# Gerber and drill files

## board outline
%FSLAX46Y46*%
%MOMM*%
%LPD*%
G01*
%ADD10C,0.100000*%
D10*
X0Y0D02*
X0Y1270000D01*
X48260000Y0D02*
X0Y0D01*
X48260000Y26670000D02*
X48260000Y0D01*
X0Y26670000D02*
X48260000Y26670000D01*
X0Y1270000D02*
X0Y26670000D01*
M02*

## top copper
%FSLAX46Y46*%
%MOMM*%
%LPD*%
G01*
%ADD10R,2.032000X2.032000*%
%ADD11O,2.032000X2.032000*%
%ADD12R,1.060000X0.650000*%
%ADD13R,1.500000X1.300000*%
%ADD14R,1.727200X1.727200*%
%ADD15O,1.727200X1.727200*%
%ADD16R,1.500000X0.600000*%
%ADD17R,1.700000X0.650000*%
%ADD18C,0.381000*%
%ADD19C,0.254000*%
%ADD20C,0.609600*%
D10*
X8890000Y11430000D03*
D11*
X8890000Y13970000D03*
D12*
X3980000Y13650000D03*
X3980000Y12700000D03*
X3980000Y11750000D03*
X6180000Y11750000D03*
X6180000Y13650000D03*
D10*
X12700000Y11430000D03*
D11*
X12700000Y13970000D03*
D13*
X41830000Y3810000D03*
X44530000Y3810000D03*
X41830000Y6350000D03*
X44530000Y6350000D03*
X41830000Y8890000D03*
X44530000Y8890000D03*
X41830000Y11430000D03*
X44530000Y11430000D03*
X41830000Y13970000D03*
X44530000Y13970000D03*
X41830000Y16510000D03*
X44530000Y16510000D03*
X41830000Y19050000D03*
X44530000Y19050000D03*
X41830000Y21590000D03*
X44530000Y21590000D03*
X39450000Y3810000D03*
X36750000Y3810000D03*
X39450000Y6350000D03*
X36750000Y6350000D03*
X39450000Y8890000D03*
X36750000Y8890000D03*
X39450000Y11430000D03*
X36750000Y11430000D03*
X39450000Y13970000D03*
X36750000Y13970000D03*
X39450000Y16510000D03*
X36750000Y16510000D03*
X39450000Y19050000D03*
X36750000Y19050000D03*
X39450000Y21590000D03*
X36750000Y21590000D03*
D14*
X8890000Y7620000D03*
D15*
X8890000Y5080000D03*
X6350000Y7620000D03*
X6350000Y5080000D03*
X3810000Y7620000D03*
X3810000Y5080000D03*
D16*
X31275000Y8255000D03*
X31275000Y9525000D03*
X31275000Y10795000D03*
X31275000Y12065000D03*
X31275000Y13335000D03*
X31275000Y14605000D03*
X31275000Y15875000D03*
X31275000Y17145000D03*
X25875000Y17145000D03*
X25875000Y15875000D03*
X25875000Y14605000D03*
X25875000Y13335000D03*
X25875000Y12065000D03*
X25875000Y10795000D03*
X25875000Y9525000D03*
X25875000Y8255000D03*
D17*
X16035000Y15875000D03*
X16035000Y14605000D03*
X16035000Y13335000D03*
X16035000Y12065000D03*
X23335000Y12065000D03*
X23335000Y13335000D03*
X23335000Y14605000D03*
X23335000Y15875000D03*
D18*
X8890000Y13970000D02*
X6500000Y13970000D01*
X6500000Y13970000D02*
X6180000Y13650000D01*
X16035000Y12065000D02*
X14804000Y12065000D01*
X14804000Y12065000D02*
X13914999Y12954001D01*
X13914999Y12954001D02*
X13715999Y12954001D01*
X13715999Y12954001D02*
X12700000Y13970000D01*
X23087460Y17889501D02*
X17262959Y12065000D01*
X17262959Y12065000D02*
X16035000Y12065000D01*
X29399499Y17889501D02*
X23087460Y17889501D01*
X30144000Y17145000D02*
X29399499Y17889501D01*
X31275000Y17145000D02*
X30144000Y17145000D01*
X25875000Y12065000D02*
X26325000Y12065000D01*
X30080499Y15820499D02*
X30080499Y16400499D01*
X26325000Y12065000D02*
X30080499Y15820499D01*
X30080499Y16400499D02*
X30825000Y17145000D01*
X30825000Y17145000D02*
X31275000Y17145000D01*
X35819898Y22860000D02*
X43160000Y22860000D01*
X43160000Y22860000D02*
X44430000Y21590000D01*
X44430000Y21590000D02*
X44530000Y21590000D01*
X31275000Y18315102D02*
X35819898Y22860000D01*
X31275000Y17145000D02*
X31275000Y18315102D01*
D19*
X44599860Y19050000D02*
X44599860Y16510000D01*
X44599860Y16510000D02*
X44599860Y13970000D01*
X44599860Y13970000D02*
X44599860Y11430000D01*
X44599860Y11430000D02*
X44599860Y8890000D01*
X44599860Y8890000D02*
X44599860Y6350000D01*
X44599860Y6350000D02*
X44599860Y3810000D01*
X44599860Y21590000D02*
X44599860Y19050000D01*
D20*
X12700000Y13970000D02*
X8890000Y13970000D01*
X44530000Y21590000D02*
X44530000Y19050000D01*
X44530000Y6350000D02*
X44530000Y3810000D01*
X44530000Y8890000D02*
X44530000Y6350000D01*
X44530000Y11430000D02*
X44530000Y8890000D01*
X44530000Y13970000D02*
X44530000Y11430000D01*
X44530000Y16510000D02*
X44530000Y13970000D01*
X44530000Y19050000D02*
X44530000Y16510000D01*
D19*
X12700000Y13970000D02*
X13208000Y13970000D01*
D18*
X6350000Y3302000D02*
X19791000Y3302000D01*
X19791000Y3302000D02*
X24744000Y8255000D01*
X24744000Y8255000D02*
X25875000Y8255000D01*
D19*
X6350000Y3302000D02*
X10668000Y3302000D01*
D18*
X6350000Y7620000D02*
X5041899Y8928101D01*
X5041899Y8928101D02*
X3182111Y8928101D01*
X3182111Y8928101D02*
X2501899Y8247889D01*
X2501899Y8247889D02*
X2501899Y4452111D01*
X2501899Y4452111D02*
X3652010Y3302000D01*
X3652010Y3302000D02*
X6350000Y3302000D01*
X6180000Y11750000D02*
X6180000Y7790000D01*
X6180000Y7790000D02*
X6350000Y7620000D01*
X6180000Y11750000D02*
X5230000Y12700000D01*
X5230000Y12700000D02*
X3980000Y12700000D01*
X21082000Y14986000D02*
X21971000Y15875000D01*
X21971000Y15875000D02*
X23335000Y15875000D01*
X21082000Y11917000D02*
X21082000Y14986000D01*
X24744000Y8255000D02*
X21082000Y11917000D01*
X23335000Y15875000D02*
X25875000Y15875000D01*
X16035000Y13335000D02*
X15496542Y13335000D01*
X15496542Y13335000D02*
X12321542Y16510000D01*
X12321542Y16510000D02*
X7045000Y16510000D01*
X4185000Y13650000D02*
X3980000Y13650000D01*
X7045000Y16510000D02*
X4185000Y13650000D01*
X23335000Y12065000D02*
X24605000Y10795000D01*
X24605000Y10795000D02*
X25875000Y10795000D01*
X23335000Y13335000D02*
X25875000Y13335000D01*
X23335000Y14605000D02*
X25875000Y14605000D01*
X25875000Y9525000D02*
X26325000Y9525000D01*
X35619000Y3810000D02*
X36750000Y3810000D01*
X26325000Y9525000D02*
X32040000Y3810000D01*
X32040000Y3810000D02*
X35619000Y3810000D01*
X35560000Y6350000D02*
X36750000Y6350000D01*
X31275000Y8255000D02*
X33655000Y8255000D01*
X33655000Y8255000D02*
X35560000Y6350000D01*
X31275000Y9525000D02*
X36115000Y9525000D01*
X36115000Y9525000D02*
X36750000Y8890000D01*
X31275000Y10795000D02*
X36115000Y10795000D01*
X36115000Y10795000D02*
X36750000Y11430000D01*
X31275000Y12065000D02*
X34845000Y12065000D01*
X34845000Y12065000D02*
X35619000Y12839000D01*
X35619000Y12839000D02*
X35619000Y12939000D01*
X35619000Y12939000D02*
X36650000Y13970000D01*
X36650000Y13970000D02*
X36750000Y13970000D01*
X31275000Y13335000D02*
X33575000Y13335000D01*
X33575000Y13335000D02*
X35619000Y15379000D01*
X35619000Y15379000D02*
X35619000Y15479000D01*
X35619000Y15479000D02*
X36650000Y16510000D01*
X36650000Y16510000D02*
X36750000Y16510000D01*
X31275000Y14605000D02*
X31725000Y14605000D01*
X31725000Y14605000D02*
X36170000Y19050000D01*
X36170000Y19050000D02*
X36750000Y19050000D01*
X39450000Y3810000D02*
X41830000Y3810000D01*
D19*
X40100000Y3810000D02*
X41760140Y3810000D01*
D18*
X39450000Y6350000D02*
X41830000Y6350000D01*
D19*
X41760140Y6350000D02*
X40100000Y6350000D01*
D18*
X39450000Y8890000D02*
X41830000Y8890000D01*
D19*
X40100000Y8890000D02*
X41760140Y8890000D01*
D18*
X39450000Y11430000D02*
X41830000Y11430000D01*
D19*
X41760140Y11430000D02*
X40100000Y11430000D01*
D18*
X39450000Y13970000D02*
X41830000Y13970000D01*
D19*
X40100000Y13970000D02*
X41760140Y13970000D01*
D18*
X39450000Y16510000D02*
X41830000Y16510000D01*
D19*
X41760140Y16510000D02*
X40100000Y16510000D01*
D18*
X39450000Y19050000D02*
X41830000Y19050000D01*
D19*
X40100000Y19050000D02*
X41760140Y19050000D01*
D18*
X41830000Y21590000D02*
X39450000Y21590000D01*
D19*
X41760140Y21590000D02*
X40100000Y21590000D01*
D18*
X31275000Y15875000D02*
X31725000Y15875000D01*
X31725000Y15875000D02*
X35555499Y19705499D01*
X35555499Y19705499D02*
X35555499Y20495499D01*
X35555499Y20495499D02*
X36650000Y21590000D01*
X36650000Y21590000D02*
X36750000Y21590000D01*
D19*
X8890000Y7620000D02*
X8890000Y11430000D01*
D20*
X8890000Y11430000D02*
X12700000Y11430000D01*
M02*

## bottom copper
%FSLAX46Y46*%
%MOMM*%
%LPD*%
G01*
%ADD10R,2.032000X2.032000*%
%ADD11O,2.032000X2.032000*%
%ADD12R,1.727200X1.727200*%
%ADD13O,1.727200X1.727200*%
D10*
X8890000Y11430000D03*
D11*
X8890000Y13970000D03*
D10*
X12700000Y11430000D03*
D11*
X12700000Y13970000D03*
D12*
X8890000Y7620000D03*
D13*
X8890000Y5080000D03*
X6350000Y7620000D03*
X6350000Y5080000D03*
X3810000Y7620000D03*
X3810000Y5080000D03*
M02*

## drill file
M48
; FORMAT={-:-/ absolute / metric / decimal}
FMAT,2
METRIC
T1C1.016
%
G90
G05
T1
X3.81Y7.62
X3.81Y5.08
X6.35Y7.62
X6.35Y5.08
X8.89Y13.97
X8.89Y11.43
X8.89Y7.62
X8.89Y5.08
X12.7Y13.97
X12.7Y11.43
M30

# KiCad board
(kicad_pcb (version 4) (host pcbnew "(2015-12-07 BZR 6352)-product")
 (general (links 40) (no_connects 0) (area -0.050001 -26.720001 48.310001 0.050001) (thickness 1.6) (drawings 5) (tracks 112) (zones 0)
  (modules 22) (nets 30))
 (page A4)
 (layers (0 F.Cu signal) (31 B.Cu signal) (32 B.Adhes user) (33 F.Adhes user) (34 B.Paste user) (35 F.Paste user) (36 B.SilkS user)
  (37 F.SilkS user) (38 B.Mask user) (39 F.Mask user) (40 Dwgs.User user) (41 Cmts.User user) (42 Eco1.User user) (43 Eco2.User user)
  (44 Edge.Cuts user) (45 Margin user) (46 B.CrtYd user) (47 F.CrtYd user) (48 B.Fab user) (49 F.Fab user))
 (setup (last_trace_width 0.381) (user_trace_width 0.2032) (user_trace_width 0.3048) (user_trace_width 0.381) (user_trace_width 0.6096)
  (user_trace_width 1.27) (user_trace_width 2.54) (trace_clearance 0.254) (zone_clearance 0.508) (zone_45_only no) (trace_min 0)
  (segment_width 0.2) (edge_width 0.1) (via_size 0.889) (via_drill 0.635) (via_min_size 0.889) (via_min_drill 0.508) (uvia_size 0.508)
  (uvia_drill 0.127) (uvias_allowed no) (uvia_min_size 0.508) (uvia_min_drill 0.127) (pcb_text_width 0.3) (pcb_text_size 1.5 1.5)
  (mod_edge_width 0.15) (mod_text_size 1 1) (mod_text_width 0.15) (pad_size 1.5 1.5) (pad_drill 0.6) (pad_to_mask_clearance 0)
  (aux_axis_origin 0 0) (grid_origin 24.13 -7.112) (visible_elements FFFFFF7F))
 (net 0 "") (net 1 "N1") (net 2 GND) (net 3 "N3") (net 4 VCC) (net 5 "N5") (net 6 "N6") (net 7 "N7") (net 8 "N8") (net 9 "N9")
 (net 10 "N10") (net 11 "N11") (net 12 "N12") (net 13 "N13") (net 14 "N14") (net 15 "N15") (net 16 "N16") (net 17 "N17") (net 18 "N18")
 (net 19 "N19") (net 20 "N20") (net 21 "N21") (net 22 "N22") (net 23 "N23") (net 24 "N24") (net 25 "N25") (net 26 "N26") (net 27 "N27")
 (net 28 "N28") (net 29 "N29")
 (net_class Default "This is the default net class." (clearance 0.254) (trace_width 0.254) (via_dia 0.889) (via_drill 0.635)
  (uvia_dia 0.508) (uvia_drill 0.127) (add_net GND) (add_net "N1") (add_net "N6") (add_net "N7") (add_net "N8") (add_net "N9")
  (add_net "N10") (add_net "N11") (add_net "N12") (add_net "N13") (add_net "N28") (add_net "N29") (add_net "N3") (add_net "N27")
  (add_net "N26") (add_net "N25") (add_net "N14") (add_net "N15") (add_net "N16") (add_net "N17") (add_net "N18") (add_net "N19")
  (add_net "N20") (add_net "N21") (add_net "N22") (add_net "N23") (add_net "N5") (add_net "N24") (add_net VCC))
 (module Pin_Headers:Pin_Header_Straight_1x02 (layer F.Cu) (at 8.89 -11.43 180)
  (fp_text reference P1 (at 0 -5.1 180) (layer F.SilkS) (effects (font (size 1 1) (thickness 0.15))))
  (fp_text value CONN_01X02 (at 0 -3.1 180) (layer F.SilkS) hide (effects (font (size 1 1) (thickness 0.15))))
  (pad 1 thru_hole rect (at 0 0 180) (size 2.032 2.032) (drill 1.016) (layers *.Cu *.Mask F.SilkS) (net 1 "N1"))
  (pad 2 thru_hole oval (at 0 2.54 180) (size 2.032 2.032) (drill 1.016) (layers *.Cu *.Mask F.SilkS) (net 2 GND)))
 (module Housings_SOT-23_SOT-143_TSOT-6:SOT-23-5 (layer F.Cu) (at 5.08 -12.7)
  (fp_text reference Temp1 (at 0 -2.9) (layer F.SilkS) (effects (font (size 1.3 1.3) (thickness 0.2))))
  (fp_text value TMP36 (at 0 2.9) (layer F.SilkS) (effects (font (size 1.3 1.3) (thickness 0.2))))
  (pad 1 smd rect (at -1.1 -0.95) (size 1.06 0.65) (layers F.Cu F.Paste F.Mask) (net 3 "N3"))
  (pad 2 smd rect (at -1.1 0) (size 1.06 0.65) (layers F.Cu F.Paste F.Mask) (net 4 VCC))
  (pad 3 smd rect (at -1.1 0.95) (size 1.06 0.65) (layers F.Cu F.Paste F.Mask) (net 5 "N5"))
  (pad 4 smd rect (at 1.1 0.95) (size 1.06 0.65) (layers F.Cu F.Paste F.Mask) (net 4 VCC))
  (pad 5 smd rect (at 1.1 -0.95) (size 1.06 0.65) (layers F.Cu F.Paste F.Mask) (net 2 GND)))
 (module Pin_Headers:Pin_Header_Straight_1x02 (layer F.Cu) (at 12.7 -11.43 180)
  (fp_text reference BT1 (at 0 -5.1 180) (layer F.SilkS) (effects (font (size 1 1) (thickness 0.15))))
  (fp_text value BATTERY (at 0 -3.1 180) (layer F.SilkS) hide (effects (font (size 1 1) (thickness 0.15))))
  (pad 1 thru_hole rect (at 0 0 180) (size 2.032 2.032) (drill 1.016) (layers *.Cu *.Mask F.SilkS) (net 1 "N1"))
  (pad 2 thru_hole oval (at 0 2.54 180) (size 2.032 2.032) (drill 1.016) (layers *.Cu *.Mask F.SilkS) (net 2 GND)))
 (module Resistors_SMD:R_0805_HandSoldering (layer F.Cu) (at 43.18 -3.81)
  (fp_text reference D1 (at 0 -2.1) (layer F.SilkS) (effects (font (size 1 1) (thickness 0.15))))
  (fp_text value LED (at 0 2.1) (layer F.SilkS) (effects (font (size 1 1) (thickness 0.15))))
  (pad 1 smd rect (at -1.35 0) (size 1.5 1.3) (layers F.Cu F.Paste F.Mask) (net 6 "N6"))
  (pad 2 smd rect (at 1.35 0) (size 1.5 1.3) (layers F.Cu F.Paste F.Mask) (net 2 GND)))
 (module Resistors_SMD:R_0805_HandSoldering (layer F.Cu) (at 43.18 -6.35)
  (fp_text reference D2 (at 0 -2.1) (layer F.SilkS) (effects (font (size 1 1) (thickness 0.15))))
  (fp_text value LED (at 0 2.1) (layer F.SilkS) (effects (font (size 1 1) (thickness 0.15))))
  (pad 1 smd rect (at -1.35 0) (size 1.5 1.3) (layers F.Cu F.Paste F.Mask) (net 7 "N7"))
  (pad 2 smd rect (at 1.35 0) (size 1.5 1.3) (layers F.Cu F.Paste F.Mask) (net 2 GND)))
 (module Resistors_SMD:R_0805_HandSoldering (layer F.Cu) (at 43.18 -8.89)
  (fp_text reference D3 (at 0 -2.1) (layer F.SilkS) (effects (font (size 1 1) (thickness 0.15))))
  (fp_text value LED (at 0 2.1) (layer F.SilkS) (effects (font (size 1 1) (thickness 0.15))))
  (pad 1 smd rect (at -1.35 0) (size 1.5 1.3) (layers F.Cu F.Paste F.Mask) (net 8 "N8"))
  (pad 2 smd rect (at 1.35 0) (size 1.5 1.3) (layers F.Cu F.Paste F.Mask) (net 2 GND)))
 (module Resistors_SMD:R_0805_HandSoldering (layer F.Cu) (at 43.18 -11.43)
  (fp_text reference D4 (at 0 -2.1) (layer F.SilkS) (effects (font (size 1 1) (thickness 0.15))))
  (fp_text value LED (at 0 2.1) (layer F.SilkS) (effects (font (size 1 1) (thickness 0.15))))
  (pad 1 smd rect (at -1.35 0) (size 1.5 1.3) (layers F.Cu F.Paste F.Mask) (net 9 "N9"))
  (pad 2 smd rect (at 1.35 0) (size 1.5 1.3) (layers F.Cu F.Paste F.Mask) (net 2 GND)))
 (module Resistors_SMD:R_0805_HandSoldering (layer F.Cu) (at 43.18 -13.97)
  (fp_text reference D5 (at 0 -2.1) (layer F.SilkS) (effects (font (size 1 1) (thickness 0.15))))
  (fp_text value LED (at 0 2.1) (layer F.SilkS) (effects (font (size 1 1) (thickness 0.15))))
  (pad 1 smd rect (at -1.35 0) (size 1.5 1.3) (layers F.Cu F.Paste F.Mask) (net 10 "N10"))
  (pad 2 smd rect (at 1.35 0) (size 1.5 1.3) (layers F.Cu F.Paste F.Mask) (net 2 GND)))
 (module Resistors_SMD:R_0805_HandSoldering (layer F.Cu) (at 43.18 -16.51)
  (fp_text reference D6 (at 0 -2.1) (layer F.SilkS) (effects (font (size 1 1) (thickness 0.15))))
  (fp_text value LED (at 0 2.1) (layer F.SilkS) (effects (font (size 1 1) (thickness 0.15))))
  (pad 1 smd rect (at -1.35 0) (size 1.5 1.3) (layers F.Cu F.Paste F.Mask) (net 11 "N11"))
  (pad 2 smd rect (at 1.35 0) (size 1.5 1.3) (layers F.Cu F.Paste F.Mask) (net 2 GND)))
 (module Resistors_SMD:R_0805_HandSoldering (layer F.Cu) (at 43.18 -19.05)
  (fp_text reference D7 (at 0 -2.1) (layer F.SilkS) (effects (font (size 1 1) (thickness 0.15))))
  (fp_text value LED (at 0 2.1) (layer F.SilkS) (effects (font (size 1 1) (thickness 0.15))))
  (pad 1 smd rect (at -1.35 0) (size 1.5 1.3) (layers F.Cu F.Paste F.Mask) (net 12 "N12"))
  (pad 2 smd rect (at 1.35 0) (size 1.5 1.3) (layers F.Cu F.Paste F.Mask) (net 2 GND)))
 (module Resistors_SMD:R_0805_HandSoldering (layer F.Cu) (at 43.18 -21.59)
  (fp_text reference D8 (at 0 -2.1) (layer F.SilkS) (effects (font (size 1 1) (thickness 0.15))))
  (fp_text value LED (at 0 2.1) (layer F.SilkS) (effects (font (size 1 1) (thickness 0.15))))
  (pad 1 smd rect (at -1.35 0) (size 1.5 1.3) (layers F.Cu F.Paste F.Mask) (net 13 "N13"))
  (pad 2 smd rect (at 1.35 0) (size 1.5 1.3) (layers F.Cu F.Paste F.Mask) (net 2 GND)))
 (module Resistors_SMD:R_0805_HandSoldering (layer F.Cu) (at 38.1 -3.81 180)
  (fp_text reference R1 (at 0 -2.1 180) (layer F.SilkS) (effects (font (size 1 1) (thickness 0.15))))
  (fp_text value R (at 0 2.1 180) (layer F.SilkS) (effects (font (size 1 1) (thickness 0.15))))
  (pad 1 smd rect (at -1.35 0 180) (size 1.5 1.3) (layers F.Cu F.Paste F.Mask) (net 6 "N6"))
  (pad 2 smd rect (at 1.35 0 180) (size 1.5 1.3) (layers F.Cu F.Paste F.Mask) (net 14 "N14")))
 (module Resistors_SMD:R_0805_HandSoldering (layer F.Cu) (at 38.1 -6.35 180)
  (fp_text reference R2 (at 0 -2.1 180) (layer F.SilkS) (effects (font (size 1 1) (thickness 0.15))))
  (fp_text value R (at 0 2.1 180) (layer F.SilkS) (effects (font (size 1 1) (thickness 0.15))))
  (pad 1 smd rect (at -1.35 0 180) (size 1.5 1.3) (layers F.Cu F.Paste F.Mask) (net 7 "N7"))
  (pad 2 smd rect (at 1.35 0 180) (size 1.5 1.3) (layers F.Cu F.Paste F.Mask) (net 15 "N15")))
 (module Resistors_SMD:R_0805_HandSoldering (layer F.Cu) (at 38.1 -8.89 180)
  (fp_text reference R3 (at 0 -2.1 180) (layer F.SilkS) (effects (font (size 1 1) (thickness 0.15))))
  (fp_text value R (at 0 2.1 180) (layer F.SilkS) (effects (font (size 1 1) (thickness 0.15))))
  (pad 1 smd rect (at -1.35 0 180) (size 1.5 1.3) (layers F.Cu F.Paste F.Mask) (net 8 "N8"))
  (pad 2 smd rect (at 1.35 0 180) (size 1.5 1.3) (layers F.Cu F.Paste F.Mask) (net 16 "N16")))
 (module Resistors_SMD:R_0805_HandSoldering (layer F.Cu) (at 38.1 -11.43 180)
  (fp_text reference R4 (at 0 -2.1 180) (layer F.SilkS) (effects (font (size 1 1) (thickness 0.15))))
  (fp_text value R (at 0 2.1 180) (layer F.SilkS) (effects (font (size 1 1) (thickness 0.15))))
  (pad 1 smd rect (at -1.35 0 180) (size 1.5 1.3) (layers F.Cu F.Paste F.Mask) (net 9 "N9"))
  (pad 2 smd rect (at 1.35 0 180) (size 1.5 1.3) (layers F.Cu F.Paste F.Mask) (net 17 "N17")))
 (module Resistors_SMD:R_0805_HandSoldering (layer F.Cu) (at 38.1 -13.97 180)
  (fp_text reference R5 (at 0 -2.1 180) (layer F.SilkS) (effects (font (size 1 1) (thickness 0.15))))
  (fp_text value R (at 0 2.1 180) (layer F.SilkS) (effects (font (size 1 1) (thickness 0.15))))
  (pad 1 smd rect (at -1.35 0 180) (size 1.5 1.3) (layers F.Cu F.Paste F.Mask) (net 10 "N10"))
  (pad 2 smd rect (at 1.35 0 180) (size 1.5 1.3) (layers F.Cu F.Paste F.Mask) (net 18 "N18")))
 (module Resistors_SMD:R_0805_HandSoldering (layer F.Cu) (at 38.1 -16.51 180)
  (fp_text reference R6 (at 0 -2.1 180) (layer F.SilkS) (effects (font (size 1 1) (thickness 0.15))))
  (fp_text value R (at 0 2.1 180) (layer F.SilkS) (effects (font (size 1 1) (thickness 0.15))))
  (pad 1 smd rect (at -1.35 0 180) (size 1.5 1.3) (layers F.Cu F.Paste F.Mask) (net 11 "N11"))
  (pad 2 smd rect (at 1.35 0 180) (size 1.5 1.3) (layers F.Cu F.Paste F.Mask) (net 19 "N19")))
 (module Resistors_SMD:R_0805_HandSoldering (layer F.Cu) (at 38.1 -19.05 180)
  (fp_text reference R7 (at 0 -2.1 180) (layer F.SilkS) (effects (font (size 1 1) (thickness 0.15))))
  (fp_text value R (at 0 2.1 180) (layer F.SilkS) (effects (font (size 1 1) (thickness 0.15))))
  (pad 1 smd rect (at -1.35 0 180) (size 1.5 1.3) (layers F.Cu F.Paste F.Mask) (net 12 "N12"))
  (pad 2 smd rect (at 1.35 0 180) (size 1.5 1.3) (layers F.Cu F.Paste F.Mask) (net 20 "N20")))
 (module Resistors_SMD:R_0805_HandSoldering (layer F.Cu) (at 38.1 -21.59 180)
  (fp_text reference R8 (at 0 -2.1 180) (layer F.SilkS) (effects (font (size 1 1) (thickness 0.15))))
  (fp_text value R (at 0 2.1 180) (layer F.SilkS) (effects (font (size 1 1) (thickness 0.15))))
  (pad 1 smd rect (at -1.35 0 180) (size 1.5 1.3) (layers F.Cu F.Paste F.Mask) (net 13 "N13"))
  (pad 2 smd rect (at 1.35 0 180) (size 1.5 1.3) (layers F.Cu F.Paste F.Mask) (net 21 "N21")))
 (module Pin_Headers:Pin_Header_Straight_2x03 (layer F.Cu) (at 8.89 -7.62 270)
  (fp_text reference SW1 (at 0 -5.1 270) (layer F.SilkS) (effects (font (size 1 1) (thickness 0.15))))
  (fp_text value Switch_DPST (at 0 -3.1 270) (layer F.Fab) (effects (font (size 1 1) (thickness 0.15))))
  (pad 1 thru_hole rect (at 0 0 270) (size 1.7272 1.7272) (drill 1.016) (layers *.Cu *.Mask F.SilkS) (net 1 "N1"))
  (pad 2 thru_hole oval (at 2.54 0 270) (size 1.7272 1.7272) (drill 1.016) (layers *.Cu *.Mask F.SilkS) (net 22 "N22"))
  (pad 3 thru_hole oval (at 0 2.54 270) (size 1.7272 1.7272) (drill 1.016) (layers *.Cu *.Mask F.SilkS) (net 4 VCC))
  (pad 4 thru_hole oval (at 2.54 2.54 270) (size 1.7272 1.7272) (drill 1.016) (layers *.Cu *.Mask F.SilkS) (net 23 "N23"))
  (pad 5 thru_hole oval (at 0 5.08 270) (size 1.7272 1.7272) (drill 1.016) (layers *.Cu *.Mask F.SilkS))
  (pad 6 thru_hole oval (at 2.54 5.08 270) (size 1.7272 1.7272) (drill 1.016) (layers *.Cu *.Mask F.SilkS)))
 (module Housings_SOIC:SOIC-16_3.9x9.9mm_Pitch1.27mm (layer F.Cu) (at 28.575 -12.7 180)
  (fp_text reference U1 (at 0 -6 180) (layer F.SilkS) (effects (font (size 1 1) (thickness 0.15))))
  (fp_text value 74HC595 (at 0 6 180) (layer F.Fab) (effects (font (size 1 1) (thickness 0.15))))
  (pad 1 smd rect (at -2.7 -4.445 180) (size 1.5 0.6) (layers F.Cu F.Paste F.Mask) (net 15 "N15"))
  (pad 2 smd rect (at -2.7 -3.175 180) (size 1.5 0.6) (layers F.Cu F.Paste F.Mask) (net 16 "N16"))
  (pad 3 smd rect (at -2.7 -1.905 180) (size 1.5 0.6) (layers F.Cu F.Paste F.Mask) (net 17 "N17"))
  (pad 4 smd rect (at -2.7 -0.635 180) (size 1.5 0.6) (layers F.Cu F.Paste F.Mask) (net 18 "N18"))
  (pad 5 smd rect (at -2.7 0.635 180) (size 1.5 0.6) (layers F.Cu F.Paste F.Mask) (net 19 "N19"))
  (pad 6 smd rect (at -2.7 1.905 180) (size 1.5 0.6) (layers F.Cu F.Paste F.Mask) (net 20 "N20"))
  (pad 7 smd rect (at -2.7 3.175 180) (size 1.5 0.6) (layers F.Cu F.Paste F.Mask) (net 21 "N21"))
  (pad 8 smd rect (at -2.7 4.445 180) (size 1.5 0.6) (layers F.Cu F.Paste F.Mask) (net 2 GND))
  (pad 9 smd rect (at 2.7 4.445 180) (size 1.5 0.6) (layers F.Cu F.Paste F.Mask) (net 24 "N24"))
  (pad 10 smd rect (at 2.7 3.175 180) (size 1.5 0.6) (layers F.Cu F.Paste F.Mask) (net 4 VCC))
  (pad 11 smd rect (at 2.7 1.905 180) (size 1.5 0.6) (layers F.Cu F.Paste F.Mask) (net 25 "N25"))
  (pad 12 smd rect (at 2.7 0.635 180) (size 1.5 0.6) (layers F.Cu F.Paste F.Mask) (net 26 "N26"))
  (pad 13 smd rect (at 2.7 -0.635 180) (size 1.5 0.6) (layers F.Cu F.Paste F.Mask) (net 2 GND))
  (pad 14 smd rect (at 2.7 -1.905 180) (size 1.5 0.6) (layers F.Cu F.Paste F.Mask) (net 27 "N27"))
  (pad 15 smd rect (at 2.7 -3.175 180) (size 1.5 0.6) (layers F.Cu F.Paste F.Mask) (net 14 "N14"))
  (pad 16 smd rect (at 2.7 -4.445 180) (size 1.5 0.6) (layers F.Cu F.Paste F.Mask) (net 4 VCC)))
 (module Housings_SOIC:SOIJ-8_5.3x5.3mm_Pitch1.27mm (layer F.Cu) (at 19.685 -13.97)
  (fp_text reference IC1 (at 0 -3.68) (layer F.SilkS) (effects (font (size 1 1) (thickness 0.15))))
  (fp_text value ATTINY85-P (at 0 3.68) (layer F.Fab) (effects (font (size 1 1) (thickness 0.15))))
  (pad 1 smd rect (at -3.65 -1.905) (size 1.7 0.65) (layers F.Cu F.Paste F.Mask) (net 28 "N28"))
  (pad 2 smd rect (at -3.65 -0.635) (size 1.7 0.65) (layers F.Cu F.Paste F.Mask) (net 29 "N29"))
  (pad 3 smd rect (at -3.65 0.635) (size 1.7 0.65) (layers F.Cu F.Paste F.Mask) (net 3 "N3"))
  (pad 4 smd rect (at -3.65 1.905) (size 1.7 0.65) (layers F.Cu F.Paste F.Mask) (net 2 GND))
  (pad 5 smd rect (at 3.65 1.905) (size 1.7 0.65) (layers F.Cu F.Paste F.Mask) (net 27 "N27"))
  (pad 6 smd rect (at 3.65 0.635) (size 1.7 0.65) (layers F.Cu F.Paste F.Mask) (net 26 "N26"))
  (pad 7 smd rect (at 3.65 -0.635) (size 1.7 0.65) (layers F.Cu F.Paste F.Mask) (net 25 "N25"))
  (pad 8 smd rect (at 3.65 -1.905) (size 1.7 0.65) (layers F.Cu F.Paste F.Mask) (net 4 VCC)))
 (gr_line (start 0 0) (end 0 -1.27) (angle 90) (layer Edge.Cuts) (width 0.1))
 (gr_line (start 48.26 0) (end 0 0) (angle 90) (layer Edge.Cuts) (width 0.1))
 (gr_line (start 48.26 -26.67) (end 48.26 0) (angle 90) (layer Edge.Cuts) (width 0.1))
 (gr_line (start 0 -26.67) (end 48.26 -26.67) (angle 90) (layer Edge.Cuts) (width 0.1))
 (gr_line (start 0 -1.27) (end 0 -26.67) (angle 90) (layer Edge.Cuts) (width 0.1))
 (segment (start 8.89 -13.97) (end 6.5 -13.97) (width 0.381) (layer F.Cu) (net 2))
 (segment (start 6.5 -13.97) (end 6.18 -13.65) (width 0.381) (layer F.Cu) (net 2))
 (segment (start 16.035 -12.065) (end 14.804 -12.065) (width 0.381) (layer F.Cu) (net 2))
 (segment (start 14.804 -12.065) (end 13.914999 -12.954001) (width 0.381) (layer F.Cu) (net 2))
 (segment (start 13.914999 -12.954001) (end 13.715999 -12.954001) (width 0.381) (layer F.Cu) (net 2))
 (segment (start 13.715999 -12.954001) (end 12.7 -13.97) (width 0.381) (layer F.Cu) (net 2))
 (segment (start 23.08746 -17.889501) (end 17.262959 -12.065) (width 0.381) (layer F.Cu) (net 2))
 (segment (start 17.262959 -12.065) (end 16.035 -12.065) (width 0.381) (layer F.Cu) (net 2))
 (segment (start 29.399499 -17.889501) (end 23.08746 -17.889501) (width 0.381) (layer F.Cu) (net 2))
 (segment (start 30.144 -17.145) (end 29.399499 -17.889501) (width 0.381) (layer F.Cu) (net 2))
 (segment (start 31.275 -17.145) (end 30.144 -17.145) (width 0.381) (layer F.Cu) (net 2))
 (segment (start 25.875 -12.065) (end 26.325 -12.065) (width 0.381) (layer F.Cu) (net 2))
 (segment (start 30.080499 -15.820499) (end 30.080499 -16.400499) (width 0.381) (layer F.Cu) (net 2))
 (segment (start 26.325 -12.065) (end 30.080499 -15.820499) (width 0.381) (layer F.Cu) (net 2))
 (segment (start 30.080499 -16.400499) (end 30.825 -17.145) (width 0.381) (layer F.Cu) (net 2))
 (segment (start 30.825 -17.145) (end 31.275 -17.145) (width 0.381) (layer F.Cu) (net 2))
 (segment (start 35.819898 -22.86) (end 43.16 -22.86) (width 0.381) (layer F.Cu) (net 2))
 (segment (start 43.16 -22.86) (end 44.43 -21.59) (width 0.381) (layer F.Cu) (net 2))
 (segment (start 44.43 -21.59) (end 44.53 -21.59) (width 0.381) (layer F.Cu) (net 2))
 (segment (start 31.275 -18.315102) (end 35.819898 -22.86) (width 0.381) (layer F.Cu) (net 2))
 (segment (start 31.275 -17.145) (end 31.275 -18.315102) (width 0.381) (layer F.Cu) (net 2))
 (segment (start 44.59986 -19.05) (end 44.59986 -16.51) (width 0.254) (layer F.Cu) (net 2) (status 20))
 (segment (start 44.59986 -16.51) (end 44.59986 -13.97) (width 0.254) (layer F.Cu) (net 2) (status 20))
 (segment (start 44.59986 -13.97) (end 44.59986 -11.43) (width 0.254) (layer F.Cu) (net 2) (status 20))
 (segment (start 44.59986 -11.43) (end 44.59986 -8.89) (width 0.254) (layer F.Cu) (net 2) (status 20))
 (segment (start 44.59986 -8.89) (end 44.59986 -6.35) (width 0.254) (layer F.Cu) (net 2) (status 20))
 (segment (start 44.59986 -6.35) (end 44.59986 -3.81) (width 0.254) (layer F.Cu) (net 2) (status 20))
 (segment (start 44.59986 -21.59) (end 44.59986 -19.05) (width 0.254) (layer F.Cu) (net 2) (status 20))
 (segment (start 12.7 -13.97) (end 8.89 -13.97) (width 0.6096) (layer F.Cu) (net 2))
 (segment (start 44.53 -21.59) (end 44.53 -19.05) (width 0.6096) (layer F.Cu) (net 2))
 (segment (start 44.53 -6.35) (end 44.53 -3.81) (width 0.6096) (layer F.Cu) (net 2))
 (segment (start 44.53 -8.89) (end 44.53 -6.35) (width 0.6096) (layer F.Cu) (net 2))
 (segment (start 44.53 -11.43) (end 44.53 -8.89) (width 0.6096) (layer F.Cu) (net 2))
 (segment (start 44.53 -13.97) (end 44.53 -11.43) (width 0.6096) (layer F.Cu) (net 2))
 (segment (start 44.53 -16.51) (end 44.53 -13.97) (width 0.6096) (layer F.Cu) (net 2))
 (segment (start 44.53 -19.05) (end 44.53 -16.51) (width 0.6096) (layer F.Cu) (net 2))
 (segment (start 12.7 -13.97) (end 13.208 -13.97) (width 0.254) (layer F.Cu) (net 2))
 (segment (start 6.35 -3.302) (end 19.791 -3.302) (width 0.381) (layer F.Cu) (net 4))
 (segment (start 19.791 -3.302) (end 24.744 -8.255) (width 0.381) (layer F.Cu) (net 4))
 (segment (start 24.744 -8.255) (end 25.875 -8.255) (width 0.381) (layer F.Cu) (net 4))
 (segment (start 6.35 -3.302) (end 10.668 -3.302) (width 0.254) (layer F.Cu) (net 4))
 (segment (start 6.35 -7.62) (end 5.041899 -8.928101) (width 0.381) (layer F.Cu) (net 4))
 (segment (start 5.041899 -8.928101) (end 3.182111 -8.928101) (width 0.381) (layer F.Cu) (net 4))
 (segment (start 3.182111 -8.928101) (end 2.501899 -8.247889) (width 0.381) (layer F.Cu) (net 4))
 (segment (start 2.501899 -8.247889) (end 2.501899 -4.452111) (width 0.381) (layer F.Cu) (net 4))
 (segment (start 2.501899 -4.452111) (end 3.65201 -3.302) (width 0.381) (layer F.Cu) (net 4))
 (segment (start 3.65201 -3.302) (end 6.35 -3.302) (width 0.381) (layer F.Cu) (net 4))
 (segment (start 6.18 -11.75) (end 6.18 -7.79) (width 0.381) (layer F.Cu) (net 4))
 (segment (start 6.18 -7.79) (end 6.35 -7.62) (width 0.381) (layer F.Cu) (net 4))
 (segment (start 6.18 -11.75) (end 5.23 -12.7) (width 0.381) (layer F.Cu) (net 4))
 (segment (start 5.23 -12.7) (end 3.98 -12.7) (width 0.381) (layer F.Cu) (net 4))
 (segment (start 21.082 -14.986) (end 21.971 -15.875) (width 0.381) (layer F.Cu) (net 4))
 (segment (start 21.971 -15.875) (end 23.335 -15.875) (width 0.381) (layer F.Cu) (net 4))
 (segment (start 21.082 -11.917) (end 21.082 -14.986) (width 0.381) (layer F.Cu) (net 4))
 (segment (start 24.744 -8.255) (end 21.082 -11.917) (width 0.381) (layer F.Cu) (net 4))
 (segment (start 23.335 -15.875) (end 25.875 -15.875) (width 0.381) (layer F.Cu) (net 4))
 (segment (start 16.035 -13.335) (end 15.496542 -13.335) (width 0.381) (layer F.Cu) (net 3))
 (segment (start 15.496542 -13.335) (end 12.321542 -16.51) (width 0.381) (layer F.Cu) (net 3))
 (segment (start 12.321542 -16.51) (end 7.045 -16.51) (width 0.381) (layer F.Cu) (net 3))
 (segment (start 4.185 -13.65) (end 3.98 -13.65) (width 0.381) (layer F.Cu) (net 3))
 (segment (start 7.045 -16.51) (end 4.185 -13.65) (width 0.381) (layer F.Cu) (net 3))
 (segment (start 23.335 -12.065) (end 24.605 -10.795) (width 0.381) (layer F.Cu) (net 27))
 (segment (start 24.605 -10.795) (end 25.875 -10.795) (width 0.381) (layer F.Cu) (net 27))
 (segment (start 23.335 -13.335) (end 25.875 -13.335) (width 0.381) (layer F.Cu) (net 26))
 (segment (start 23.335 -14.605) (end 25.875 -14.605) (width 0.381) (layer F.Cu) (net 25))
 (segment (start 25.875 -9.525) (end 26.325 -9.525) (width 0.381) (layer F.Cu) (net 14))
 (segment (start 35.619 -3.81) (end 36.75 -3.81) (width 0.381) (layer F.Cu) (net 14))
 (segment (start 26.325 -9.525) (end 32.04 -3.81) (width 0.381) (layer F.Cu) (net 14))
 (segment (start 32.04 -3.81) (end 35.619 -3.81) (width 0.381) (layer F.Cu) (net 14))
 (segment (start 35.56 -6.35) (end 36.75 -6.35) (width 0.381) (layer F.Cu) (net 15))
 (segment (start 31.275 -8.255) (end 33.655 -8.255) (width 0.381) (layer F.Cu) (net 15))
 (segment (start 33.655 -8.255) (end 35.56 -6.35) (width 0.381) (layer F.Cu) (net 15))
 (segment (start 31.275 -9.525) (end 36.115 -9.525) (width 0.381) (layer F.Cu) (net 16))
 (segment (start 36.115 -9.525) (end 36.75 -8.89) (width 0.381) (layer F.Cu) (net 16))
 (segment (start 31.275 -10.795) (end 36.115 -10.795) (width 0.381) (layer F.Cu) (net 17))
 (segment (start 36.115 -10.795) (end 36.75 -11.43) (width 0.381) (layer F.Cu) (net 17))
 (segment (start 31.275 -12.065) (end 34.845 -12.065) (width 0.381) (layer F.Cu) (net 18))
 (segment (start 34.845 -12.065) (end 35.619 -12.839) (width 0.381) (layer F.Cu) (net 18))
 (segment (start 35.619 -12.839) (end 35.619 -12.939) (width 0.381) (layer F.Cu) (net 18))
 (segment (start 35.619 -12.939) (end 36.65 -13.97) (width 0.381) (layer F.Cu) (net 18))
 (segment (start 36.65 -13.97) (end 36.75 -13.97) (width 0.381) (layer F.Cu) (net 18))
 (segment (start 31.275 -13.335) (end 33.575 -13.335) (width 0.381) (layer F.Cu) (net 19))
 (segment (start 33.575 -13.335) (end 35.619 -15.379) (width 0.381) (layer F.Cu) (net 19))
 (segment (start 35.619 -15.379) (end 35.619 -15.479) (width 0.381) (layer F.Cu) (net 19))
 (segment (start 35.619 -15.479) (end 36.65 -16.51) (width 0.381) (layer F.Cu) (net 19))
 (segment (start 36.65 -16.51) (end 36.75 -16.51) (width 0.381) (layer F.Cu) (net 19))
 (segment (start 31.275 -14.605) (end 31.725 -14.605) (width 0.381) (layer F.Cu) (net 20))
 (segment (start 31.725 -14.605) (end 36.17 -19.05) (width 0.381) (layer F.Cu) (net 20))
 (segment (start 36.17 -19.05) (end 36.75 -19.05) (width 0.381) (layer F.Cu) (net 20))
 (segment (start 39.45 -3.81) (end 41.83 -3.81) (width 0.381) (layer F.Cu) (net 6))
 (segment (start 40.1 -3.81) (end 41.76014 -3.81) (width 0.254) (layer F.Cu) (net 6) (status 20))
 (segment (start 39.45 -6.35) (end 41.83 -6.35) (width 0.381) (layer F.Cu) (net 7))
 (segment (start 41.76014 -6.35) (end 40.1 -6.35) (width 0.254) (layer F.Cu) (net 7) (status 10))
 (segment (start 39.45 -8.89) (end 41.83 -8.89) (width 0.381) (layer F.Cu) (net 8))
 (segment (start 40.1 -8.89) (end 41.76014 -8.89) (width 0.254) (layer F.Cu) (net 8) (status 20))
 (segment (start 39.45 -11.43) (end 41.83 -11.43) (width 0.381) (layer F.Cu) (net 9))
 (segment (start 41.76014 -11.43) (end 40.1 -11.43) (width 0.254) (layer F.Cu) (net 9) (status 20))
 (segment (start 39.45 -13.97) (end 41.83 -13.97) (width 0.381) (layer F.Cu) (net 10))
 (segment (start 40.1 -13.97) (end 41.76014 -13.97) (width 0.254) (layer F.Cu) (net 10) (status 20))
 (segment (start 39.45 -16.51) (end 41.83 -16.51) (width 0.381) (layer F.Cu) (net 11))
 (segment (start 41.76014 -16.51) (end 40.1 -16.51) (width 0.254) (layer F.Cu) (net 11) (status 20))
 (segment (start 39.45 -19.05) (end 41.83 -19.05) (width 0.381) (layer F.Cu) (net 12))
 (segment (start 40.1 -19.05) (end 41.76014 -19.05) (width 0.254) (layer F.Cu) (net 12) (status 20))
 (segment (start 41.83 -21.59) (end 39.45 -21.59) (width 0.381) (layer F.Cu) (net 13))
 (segment (start 41.76014 -21.59) (end 40.1 -21.59) (width 0.254) (layer F.Cu) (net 13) (status 10))
 (segment (start 31.275 -15.875) (end 31.725 -15.875) (width 0.381) (layer F.Cu) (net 21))
 (segment (start 31.725 -15.875) (end 35.555499 -19.705499) (width 0.381) (layer F.Cu) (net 21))
 (segment (start 35.555499 -19.705499) (end 35.555499 -20.495499) (width 0.381) (layer F.Cu) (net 21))
 (segment (start 35.555499 -20.495499) (end 36.65 -21.59) (width 0.381) (layer F.Cu) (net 21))
 (segment (start 36.65 -21.59) (end 36.75 -21.59) (width 0.381) (layer F.Cu) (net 21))
 (segment (start 8.89 -7.62) (end 8.89 -11.43) (width 0.254) (layer F.Cu) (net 1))
 (segment (start 8.89 -11.43) (end 12.7 -11.43) (width 0.6096) (layer F.Cu) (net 1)))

